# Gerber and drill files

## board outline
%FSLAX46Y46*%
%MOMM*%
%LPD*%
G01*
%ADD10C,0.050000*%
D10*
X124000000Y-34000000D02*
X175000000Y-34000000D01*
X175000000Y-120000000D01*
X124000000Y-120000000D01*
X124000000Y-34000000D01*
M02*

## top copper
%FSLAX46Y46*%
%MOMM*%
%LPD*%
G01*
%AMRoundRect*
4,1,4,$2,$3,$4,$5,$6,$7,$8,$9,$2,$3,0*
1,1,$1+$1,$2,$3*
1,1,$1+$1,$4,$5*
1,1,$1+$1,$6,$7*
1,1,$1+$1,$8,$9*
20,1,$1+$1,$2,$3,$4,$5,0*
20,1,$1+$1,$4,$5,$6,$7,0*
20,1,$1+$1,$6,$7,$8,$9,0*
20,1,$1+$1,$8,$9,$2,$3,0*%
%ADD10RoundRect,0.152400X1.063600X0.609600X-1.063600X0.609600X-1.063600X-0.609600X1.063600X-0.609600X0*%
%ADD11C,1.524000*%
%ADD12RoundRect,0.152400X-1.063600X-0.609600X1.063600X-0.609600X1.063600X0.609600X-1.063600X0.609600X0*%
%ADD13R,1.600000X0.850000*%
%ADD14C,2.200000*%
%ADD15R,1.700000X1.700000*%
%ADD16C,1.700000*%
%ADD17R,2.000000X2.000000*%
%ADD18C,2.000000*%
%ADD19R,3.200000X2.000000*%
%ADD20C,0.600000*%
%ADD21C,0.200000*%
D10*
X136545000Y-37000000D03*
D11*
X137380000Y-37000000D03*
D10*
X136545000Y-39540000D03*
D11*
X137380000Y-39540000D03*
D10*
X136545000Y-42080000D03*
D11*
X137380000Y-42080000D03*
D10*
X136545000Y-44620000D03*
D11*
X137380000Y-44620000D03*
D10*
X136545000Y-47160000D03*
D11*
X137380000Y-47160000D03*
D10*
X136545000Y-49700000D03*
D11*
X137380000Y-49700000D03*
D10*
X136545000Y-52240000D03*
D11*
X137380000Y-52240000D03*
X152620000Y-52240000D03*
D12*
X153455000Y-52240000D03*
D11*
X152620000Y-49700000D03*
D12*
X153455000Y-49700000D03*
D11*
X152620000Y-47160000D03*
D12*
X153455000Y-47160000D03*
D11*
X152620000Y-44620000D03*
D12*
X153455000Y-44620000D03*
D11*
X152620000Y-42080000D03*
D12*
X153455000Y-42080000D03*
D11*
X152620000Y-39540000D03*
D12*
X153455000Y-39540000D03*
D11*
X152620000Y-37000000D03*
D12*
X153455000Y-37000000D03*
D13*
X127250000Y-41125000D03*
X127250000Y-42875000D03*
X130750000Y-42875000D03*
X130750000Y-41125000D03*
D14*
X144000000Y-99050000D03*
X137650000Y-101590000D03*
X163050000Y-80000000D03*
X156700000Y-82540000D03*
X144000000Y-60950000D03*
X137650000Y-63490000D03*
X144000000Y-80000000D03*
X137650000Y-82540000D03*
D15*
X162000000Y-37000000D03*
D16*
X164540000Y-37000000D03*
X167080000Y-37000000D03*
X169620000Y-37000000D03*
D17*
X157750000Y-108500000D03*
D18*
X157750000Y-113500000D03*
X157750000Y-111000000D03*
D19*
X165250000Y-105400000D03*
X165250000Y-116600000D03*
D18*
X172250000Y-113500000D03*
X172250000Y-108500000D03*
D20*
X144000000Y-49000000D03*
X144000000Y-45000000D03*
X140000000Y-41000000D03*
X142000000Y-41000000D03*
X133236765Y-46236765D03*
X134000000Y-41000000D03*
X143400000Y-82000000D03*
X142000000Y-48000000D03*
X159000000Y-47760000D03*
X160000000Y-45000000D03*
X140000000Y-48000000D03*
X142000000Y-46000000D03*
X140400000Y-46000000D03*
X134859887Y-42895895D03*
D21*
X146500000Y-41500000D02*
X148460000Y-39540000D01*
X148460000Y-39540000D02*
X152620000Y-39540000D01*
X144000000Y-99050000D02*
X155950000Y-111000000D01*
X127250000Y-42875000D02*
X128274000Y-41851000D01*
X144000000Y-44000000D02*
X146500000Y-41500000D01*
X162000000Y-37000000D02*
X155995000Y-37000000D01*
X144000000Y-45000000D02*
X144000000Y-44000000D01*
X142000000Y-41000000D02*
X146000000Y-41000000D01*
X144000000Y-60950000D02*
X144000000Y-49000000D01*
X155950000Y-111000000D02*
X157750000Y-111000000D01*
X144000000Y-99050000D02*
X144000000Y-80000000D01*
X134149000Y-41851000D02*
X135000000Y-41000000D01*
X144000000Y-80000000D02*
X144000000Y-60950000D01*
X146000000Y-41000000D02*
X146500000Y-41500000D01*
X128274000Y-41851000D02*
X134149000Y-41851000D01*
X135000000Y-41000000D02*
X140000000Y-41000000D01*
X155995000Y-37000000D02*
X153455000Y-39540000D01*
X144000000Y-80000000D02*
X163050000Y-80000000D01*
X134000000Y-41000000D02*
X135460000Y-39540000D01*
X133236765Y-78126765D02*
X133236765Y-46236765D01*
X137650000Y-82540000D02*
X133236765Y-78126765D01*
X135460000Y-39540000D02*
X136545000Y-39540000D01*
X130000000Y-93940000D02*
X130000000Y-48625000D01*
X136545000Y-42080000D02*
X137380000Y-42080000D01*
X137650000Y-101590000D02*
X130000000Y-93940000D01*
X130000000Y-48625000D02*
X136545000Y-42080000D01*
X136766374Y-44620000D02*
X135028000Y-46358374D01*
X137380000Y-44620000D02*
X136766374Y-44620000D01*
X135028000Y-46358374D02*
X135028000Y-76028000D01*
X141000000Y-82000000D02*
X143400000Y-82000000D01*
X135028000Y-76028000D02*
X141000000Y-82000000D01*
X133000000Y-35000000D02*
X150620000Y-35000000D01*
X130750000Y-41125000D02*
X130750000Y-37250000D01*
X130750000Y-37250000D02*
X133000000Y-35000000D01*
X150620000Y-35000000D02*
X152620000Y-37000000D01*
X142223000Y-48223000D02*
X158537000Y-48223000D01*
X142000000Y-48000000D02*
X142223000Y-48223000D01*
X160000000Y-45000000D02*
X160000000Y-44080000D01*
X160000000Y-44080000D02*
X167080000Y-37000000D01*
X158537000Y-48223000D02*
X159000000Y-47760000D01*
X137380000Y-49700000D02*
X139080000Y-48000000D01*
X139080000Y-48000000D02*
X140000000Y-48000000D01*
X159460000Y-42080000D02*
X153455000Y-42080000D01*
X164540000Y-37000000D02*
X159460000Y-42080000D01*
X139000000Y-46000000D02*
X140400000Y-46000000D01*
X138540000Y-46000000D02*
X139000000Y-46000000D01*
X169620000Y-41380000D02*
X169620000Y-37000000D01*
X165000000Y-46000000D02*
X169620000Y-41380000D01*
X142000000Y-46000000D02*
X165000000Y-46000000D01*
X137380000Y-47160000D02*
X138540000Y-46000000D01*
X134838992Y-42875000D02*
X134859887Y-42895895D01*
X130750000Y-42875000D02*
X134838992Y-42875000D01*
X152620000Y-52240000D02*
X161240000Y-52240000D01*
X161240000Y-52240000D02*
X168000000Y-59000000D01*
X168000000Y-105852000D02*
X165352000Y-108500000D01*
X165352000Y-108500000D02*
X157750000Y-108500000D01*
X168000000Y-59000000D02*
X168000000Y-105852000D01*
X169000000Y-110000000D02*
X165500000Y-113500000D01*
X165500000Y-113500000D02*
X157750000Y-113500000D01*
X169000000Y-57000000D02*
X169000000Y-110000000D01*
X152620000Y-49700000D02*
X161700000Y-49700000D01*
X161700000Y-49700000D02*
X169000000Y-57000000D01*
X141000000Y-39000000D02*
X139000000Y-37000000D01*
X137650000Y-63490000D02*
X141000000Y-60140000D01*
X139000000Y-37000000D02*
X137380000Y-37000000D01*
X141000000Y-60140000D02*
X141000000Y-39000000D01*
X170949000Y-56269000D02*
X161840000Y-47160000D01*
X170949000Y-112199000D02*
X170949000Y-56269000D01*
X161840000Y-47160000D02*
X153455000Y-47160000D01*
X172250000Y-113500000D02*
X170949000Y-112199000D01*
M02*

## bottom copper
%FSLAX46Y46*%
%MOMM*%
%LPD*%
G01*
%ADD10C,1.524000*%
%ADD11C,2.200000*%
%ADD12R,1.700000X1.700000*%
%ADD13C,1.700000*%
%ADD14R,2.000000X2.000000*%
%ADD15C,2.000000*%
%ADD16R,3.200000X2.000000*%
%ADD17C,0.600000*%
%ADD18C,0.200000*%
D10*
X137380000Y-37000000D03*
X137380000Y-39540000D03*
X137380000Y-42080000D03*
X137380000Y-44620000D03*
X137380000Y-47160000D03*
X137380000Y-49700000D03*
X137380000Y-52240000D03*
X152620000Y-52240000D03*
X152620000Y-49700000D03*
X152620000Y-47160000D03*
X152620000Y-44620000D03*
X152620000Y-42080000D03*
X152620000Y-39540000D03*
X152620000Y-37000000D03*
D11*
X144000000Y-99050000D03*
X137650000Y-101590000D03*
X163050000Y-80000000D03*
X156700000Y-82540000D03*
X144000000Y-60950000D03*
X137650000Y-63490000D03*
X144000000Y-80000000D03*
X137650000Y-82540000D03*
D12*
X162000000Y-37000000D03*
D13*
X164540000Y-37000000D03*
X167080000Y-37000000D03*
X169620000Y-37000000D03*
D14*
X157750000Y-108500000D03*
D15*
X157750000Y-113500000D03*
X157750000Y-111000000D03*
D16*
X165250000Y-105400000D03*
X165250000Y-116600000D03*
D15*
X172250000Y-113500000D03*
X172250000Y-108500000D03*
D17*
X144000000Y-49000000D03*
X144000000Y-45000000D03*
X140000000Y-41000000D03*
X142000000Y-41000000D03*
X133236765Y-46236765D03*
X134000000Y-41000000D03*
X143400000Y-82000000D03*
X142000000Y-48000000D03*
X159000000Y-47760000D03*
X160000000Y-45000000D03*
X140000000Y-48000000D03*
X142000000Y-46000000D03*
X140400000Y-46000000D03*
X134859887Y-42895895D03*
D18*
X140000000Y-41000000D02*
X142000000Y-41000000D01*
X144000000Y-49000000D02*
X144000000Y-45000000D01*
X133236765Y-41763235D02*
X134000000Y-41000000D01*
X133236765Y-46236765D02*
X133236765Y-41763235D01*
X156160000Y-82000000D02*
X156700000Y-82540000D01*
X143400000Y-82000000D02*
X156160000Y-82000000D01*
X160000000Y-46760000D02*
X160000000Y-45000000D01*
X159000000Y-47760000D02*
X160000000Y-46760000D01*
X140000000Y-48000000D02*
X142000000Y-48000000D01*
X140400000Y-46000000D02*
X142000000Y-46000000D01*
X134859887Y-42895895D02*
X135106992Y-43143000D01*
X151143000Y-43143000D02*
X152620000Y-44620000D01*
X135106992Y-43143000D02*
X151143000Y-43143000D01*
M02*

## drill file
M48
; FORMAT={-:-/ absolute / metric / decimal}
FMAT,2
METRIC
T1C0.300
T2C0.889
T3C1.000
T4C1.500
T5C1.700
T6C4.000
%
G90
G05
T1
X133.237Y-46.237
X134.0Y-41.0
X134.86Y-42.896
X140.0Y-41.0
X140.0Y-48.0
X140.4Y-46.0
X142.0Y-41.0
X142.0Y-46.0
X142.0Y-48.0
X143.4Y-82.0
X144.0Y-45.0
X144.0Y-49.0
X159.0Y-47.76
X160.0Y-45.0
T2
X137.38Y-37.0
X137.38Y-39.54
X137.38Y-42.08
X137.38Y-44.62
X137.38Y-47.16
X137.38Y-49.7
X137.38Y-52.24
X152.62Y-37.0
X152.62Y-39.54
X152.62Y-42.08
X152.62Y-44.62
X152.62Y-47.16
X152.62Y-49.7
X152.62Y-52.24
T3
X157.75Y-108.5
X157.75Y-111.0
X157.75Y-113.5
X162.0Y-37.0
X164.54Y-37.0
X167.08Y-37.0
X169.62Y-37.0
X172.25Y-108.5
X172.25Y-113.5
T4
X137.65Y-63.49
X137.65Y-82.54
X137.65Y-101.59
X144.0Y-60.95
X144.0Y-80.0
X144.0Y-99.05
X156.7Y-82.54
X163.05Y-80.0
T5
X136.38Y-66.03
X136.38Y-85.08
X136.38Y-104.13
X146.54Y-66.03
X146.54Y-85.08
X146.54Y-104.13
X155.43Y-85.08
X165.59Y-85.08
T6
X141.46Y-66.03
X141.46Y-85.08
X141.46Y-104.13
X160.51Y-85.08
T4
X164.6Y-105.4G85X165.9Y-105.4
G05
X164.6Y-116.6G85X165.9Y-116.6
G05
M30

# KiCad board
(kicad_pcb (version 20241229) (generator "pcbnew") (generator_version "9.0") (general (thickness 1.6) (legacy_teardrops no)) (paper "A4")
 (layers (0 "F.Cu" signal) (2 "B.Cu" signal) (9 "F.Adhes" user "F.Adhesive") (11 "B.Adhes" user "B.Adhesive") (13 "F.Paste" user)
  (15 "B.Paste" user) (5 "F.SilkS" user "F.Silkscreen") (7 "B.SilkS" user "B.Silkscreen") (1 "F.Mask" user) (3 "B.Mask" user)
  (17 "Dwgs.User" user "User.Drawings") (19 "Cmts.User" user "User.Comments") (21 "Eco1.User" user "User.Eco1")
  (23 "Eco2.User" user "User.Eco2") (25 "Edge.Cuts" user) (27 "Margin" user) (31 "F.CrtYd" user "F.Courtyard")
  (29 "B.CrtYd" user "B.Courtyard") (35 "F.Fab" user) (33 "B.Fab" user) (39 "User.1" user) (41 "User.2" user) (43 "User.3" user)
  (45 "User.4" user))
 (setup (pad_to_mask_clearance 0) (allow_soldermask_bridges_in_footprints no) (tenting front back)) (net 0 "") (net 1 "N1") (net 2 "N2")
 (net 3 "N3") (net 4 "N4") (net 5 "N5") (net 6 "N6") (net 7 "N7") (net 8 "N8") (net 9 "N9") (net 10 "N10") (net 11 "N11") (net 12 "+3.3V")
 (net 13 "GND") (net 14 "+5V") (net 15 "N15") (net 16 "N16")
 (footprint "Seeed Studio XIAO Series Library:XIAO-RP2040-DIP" (layer "F.Cu") (at 145 44.62)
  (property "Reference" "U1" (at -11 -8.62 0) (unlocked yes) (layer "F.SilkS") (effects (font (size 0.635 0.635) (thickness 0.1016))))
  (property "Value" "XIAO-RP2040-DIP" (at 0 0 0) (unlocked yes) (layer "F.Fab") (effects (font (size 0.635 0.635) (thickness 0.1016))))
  (pad "1" smd roundrect (at -8.455 -7.62 180) (size 2.432 1.524) (layers "F.Cu" "F.Mask") (roundrect_rratio 0.1) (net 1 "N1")
   (thermal_bridge_angle 45))
  (pad "1" thru_hole circle (at -7.62 -7.62 180) (size 1.524 1.524) (drill 0.889) (layers "*.Cu" "*.Mask") (remove_unused_layers no)
   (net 1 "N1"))
  (pad "2" smd roundrect (at -8.455 -5.08 180) (size 2.432 1.524) (layers "F.Cu" "F.Mask") (roundrect_rratio 0.1) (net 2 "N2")
   (thermal_bridge_angle 45))
  (pad "2" thru_hole circle (at -7.62 -5.08 180) (size 1.524 1.524) (drill 0.889) (layers "*.Cu" "*.Mask") (remove_unused_layers no)
   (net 2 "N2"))
  (pad "3" smd roundrect (at -8.455 -2.54 180) (size 2.432 1.524) (layers "F.Cu" "F.Mask") (roundrect_rratio 0.1) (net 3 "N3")
   (thermal_bridge_angle 45))
  (pad "3" thru_hole circle (at -7.62 -2.54 180) (size 1.524 1.524) (drill 0.889) (layers "*.Cu" "*.Mask") (remove_unused_layers no)
   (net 3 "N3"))
  (pad "4" smd roundrect (at -8.455 0 180) (size 2.432 1.524) (layers "F.Cu" "F.Mask") (roundrect_rratio 0.1) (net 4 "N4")
   (thermal_bridge_angle 45))
  (pad "4" thru_hole circle (at -7.62 0 180) (size 1.524 1.524) (drill 0.889) (layers "*.Cu" "*.Mask") (remove_unused_layers no)
   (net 4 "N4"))
  (pad "5" smd roundrect (at -8.455 2.54 180) (size 2.432 1.524) (layers "F.Cu" "F.Mask") (roundrect_rratio 0.1) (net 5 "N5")
   (thermal_bridge_angle 45))
  (pad "5" thru_hole circle (at -7.62 2.54 180) (size 1.524 1.524) (drill 0.889) (layers "*.Cu" "*.Mask") (remove_unused_layers no)
   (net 5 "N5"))
  (pad "6" smd roundrect (at -8.455 5.08 180) (size 2.432 1.524) (layers "F.Cu" "F.Mask") (roundrect_rratio 0.1) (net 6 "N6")
   (thermal_bridge_angle 45))
  (pad "6" thru_hole circle (at -7.62 5.08 180) (size 1.524 1.524) (drill 0.889) (layers "*.Cu" "*.Mask") (remove_unused_layers no)
   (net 6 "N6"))
  (pad "7" smd roundrect (at -8.455 7.62 180) (size 2.432 1.524) (layers "F.Cu" "F.Mask") (roundrect_rratio 0.1) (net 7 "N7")
   (thermal_bridge_angle 45))
  (pad "7" thru_hole circle (at -7.62 7.62 180) (size 1.524 1.524) (drill 0.889) (layers "*.Cu" "*.Mask") (remove_unused_layers no)
   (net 7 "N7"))
  (pad "8" thru_hole circle (at 7.62 7.62) (size 1.524 1.524) (drill 0.889) (layers "*.Cu" "*.Mask") (remove_unused_layers no) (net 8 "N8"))
  (pad "8" smd roundrect (at 8.455 7.62) (size 2.432 1.524) (layers "F.Cu" "F.Mask") (roundrect_rratio 0.1) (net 8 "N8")
   (thermal_bridge_angle 45))
  (pad "9" thru_hole circle (at 7.62 5.08) (size 1.524 1.524) (drill 0.889) (layers "*.Cu" "*.Mask") (remove_unused_layers no) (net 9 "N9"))
  (pad "9" smd roundrect (at 8.455 5.08) (size 2.432 1.524) (layers "F.Cu" "F.Mask") (roundrect_rratio 0.1) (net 9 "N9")
   (thermal_bridge_angle 45))
  (pad "10" thru_hole circle (at 7.62 2.54) (size 1.524 1.524) (drill 0.889) (layers "*.Cu" "*.Mask") (remove_unused_layers no)
   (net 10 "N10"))
  (pad "10" smd roundrect (at 8.455 2.54) (size 2.432 1.524) (layers "F.Cu" "F.Mask") (roundrect_rratio 0.1) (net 10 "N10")
   (thermal_bridge_angle 45))
  (pad "11" thru_hole circle (at 7.62 0) (size 1.524 1.524) (drill 0.889) (layers "*.Cu" "*.Mask") (remove_unused_layers no) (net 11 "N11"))
  (pad "11" smd roundrect (at 8.455 0) (size 2.432 1.524) (layers "F.Cu" "F.Mask") (roundrect_rratio 0.1) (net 11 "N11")
   (thermal_bridge_angle 45))
  (pad "12" thru_hole circle (at 7.62 -2.54) (size 1.524 1.524) (drill 0.889) (layers "*.Cu" "*.Mask") (remove_unused_layers no)
   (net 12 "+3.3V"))
  (pad "12" smd roundrect (at 8.455 -2.54) (size 2.432 1.524) (layers "F.Cu" "F.Mask") (roundrect_rratio 0.1) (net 12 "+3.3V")
   (thermal_bridge_angle 45))
  (pad "13" thru_hole circle (at 7.62 -5.08) (size 1.524 1.524) (drill 0.889) (layers "*.Cu" "*.Mask") (remove_unused_layers no)
   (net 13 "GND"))
  (pad "13" smd roundrect (at 8.455 -5.08) (size 2.432 1.524) (layers "F.Cu" "F.Mask") (roundrect_rratio 0.1) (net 13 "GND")
   (thermal_bridge_angle 45))
  (pad "14" thru_hole circle (at 7.62 -7.62) (size 1.524 1.524) (drill 0.889) (layers "*.Cu" "*.Mask") (remove_unused_layers no)
   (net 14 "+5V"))
  (pad "14" smd roundrect (at 8.455 -7.62) (size 2.432 1.524) (layers "F.Cu" "F.Mask") (roundrect_rratio 0.1) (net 14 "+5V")
   (thermal_bridge_angle 45)))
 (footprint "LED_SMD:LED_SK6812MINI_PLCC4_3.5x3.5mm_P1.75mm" (layer "F.Cu") (at 129 42)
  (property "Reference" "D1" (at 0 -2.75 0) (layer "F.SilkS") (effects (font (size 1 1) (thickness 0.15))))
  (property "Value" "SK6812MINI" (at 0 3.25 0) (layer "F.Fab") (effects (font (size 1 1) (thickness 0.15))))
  (pad "1" smd rect (at -1.75 -0.875) (size 1.6 0.85) (layers "F.Cu" "F.Mask" "F.Paste") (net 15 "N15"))
  (pad "2" smd rect (at -1.75 0.875) (size 1.6 0.85) (layers "F.Cu" "F.Mask" "F.Paste") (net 13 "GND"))
  (pad "3" smd rect (at 1.75 0.875) (size 1.6 0.85) (layers "F.Cu" "F.Mask" "F.Paste") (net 11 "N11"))
  (pad "4" smd rect (at 1.75 -0.875) (size 1.6 0.85) (layers "F.Cu" "F.Mask" "F.Paste") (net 14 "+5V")))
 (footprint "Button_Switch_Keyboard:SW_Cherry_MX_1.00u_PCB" (layer "F.Cu") (at 144 99.05)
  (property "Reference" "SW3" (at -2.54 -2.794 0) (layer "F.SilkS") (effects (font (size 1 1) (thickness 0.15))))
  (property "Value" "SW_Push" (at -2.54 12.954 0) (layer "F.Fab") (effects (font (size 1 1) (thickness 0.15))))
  (pad "" np_thru_hole circle (at -7.62 5.08) (size 1.7 1.7) (drill 1.7) (layers "*.Cu" "*.Mask"))
  (pad "" np_thru_hole circle (at -2.54 5.08) (size 4 4) (drill 4) (layers "*.Cu" "*.Mask"))
  (pad "" np_thru_hole circle (at 2.54 5.08) (size 1.7 1.7) (drill 1.7) (layers "*.Cu" "*.Mask"))
  (pad "1" thru_hole circle (at 0 0) (size 2.2 2.2) (drill 1.5) (layers "*.Cu" "*.Mask") (remove_unused_layers no) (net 13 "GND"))
  (pad "2" thru_hole circle (at -6.35 2.54) (size 2.2 2.2) (drill 1.5) (layers "*.Cu" "*.Mask") (remove_unused_layers no) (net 3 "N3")))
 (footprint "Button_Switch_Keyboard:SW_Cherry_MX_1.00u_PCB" (layer "F.Cu") (at 163.05 80)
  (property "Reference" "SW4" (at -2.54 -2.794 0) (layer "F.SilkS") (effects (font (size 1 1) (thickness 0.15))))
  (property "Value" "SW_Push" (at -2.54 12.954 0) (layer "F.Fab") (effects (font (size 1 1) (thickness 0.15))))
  (pad "" np_thru_hole circle (at -7.62 5.08) (size 1.7 1.7) (drill 1.7) (layers "*.Cu" "*.Mask"))
  (pad "" np_thru_hole circle (at -2.54 5.08) (size 4 4) (drill 4) (layers "*.Cu" "*.Mask"))
  (pad "" np_thru_hole circle (at 2.54 5.08) (size 1.7 1.7) (drill 1.7) (layers "*.Cu" "*.Mask"))
  (pad "1" thru_hole circle (at 0 0) (size 2.2 2.2) (drill 1.5) (layers "*.Cu" "*.Mask") (remove_unused_layers no) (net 13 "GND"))
  (pad "2" thru_hole circle (at -6.35 2.54) (size 2.2 2.2) (drill 1.5) (layers "*.Cu" "*.Mask") (remove_unused_layers no) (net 4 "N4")))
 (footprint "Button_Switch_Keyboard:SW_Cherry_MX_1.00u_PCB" (layer "F.Cu") (at 144 60.95)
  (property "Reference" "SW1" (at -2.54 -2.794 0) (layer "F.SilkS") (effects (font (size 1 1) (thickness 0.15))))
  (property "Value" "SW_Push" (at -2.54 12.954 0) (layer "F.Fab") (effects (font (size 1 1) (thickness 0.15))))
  (pad "" np_thru_hole circle (at -7.62 5.08) (size 1.7 1.7) (drill 1.7) (layers "*.Cu" "*.Mask"))
  (pad "" np_thru_hole circle (at -2.54 5.08) (size 4 4) (drill 4) (layers "*.Cu" "*.Mask"))
  (pad "" np_thru_hole circle (at 2.54 5.08) (size 1.7 1.7) (drill 1.7) (layers "*.Cu" "*.Mask"))
  (pad "1" thru_hole circle (at 0 0) (size 2.2 2.2) (drill 1.5) (layers "*.Cu" "*.Mask") (remove_unused_layers no) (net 13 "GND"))
  (pad "2" thru_hole circle (at -6.35 2.54) (size 2.2 2.2) (drill 1.5) (layers "*.Cu" "*.Mask") (remove_unused_layers no) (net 1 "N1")))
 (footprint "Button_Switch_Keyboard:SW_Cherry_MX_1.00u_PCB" (layer "F.Cu") (at 144 80)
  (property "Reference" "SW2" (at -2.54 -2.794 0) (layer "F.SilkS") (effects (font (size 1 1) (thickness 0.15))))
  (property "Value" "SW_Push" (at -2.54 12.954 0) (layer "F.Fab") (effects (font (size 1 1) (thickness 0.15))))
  (pad "" np_thru_hole circle (at -7.62 5.08) (size 1.7 1.7) (drill 1.7) (layers "*.Cu" "*.Mask"))
  (pad "" np_thru_hole circle (at -2.54 5.08) (size 4 4) (drill 4) (layers "*.Cu" "*.Mask"))
  (pad "" np_thru_hole circle (at 2.54 5.08) (size 1.7 1.7) (drill 1.7) (layers "*.Cu" "*.Mask"))
  (pad "1" thru_hole circle (at 0 0) (size 2.2 2.2) (drill 1.5) (layers "*.Cu" "*.Mask") (remove_unused_layers no) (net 13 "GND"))
  (pad "2" thru_hole circle (at -6.35 2.54) (size 2.2 2.2) (drill 1.5) (layers "*.Cu" "*.Mask") (remove_unused_layers no) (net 2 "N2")))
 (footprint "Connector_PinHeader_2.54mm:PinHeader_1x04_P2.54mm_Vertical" (layer "F.Cu") (at 162 37 90)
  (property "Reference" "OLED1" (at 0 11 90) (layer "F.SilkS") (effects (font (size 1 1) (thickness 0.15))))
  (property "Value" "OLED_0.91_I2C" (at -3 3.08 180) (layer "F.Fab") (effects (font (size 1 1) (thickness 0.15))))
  (pad "1" thru_hole rect (at 0 0 90) (size 1.7 1.7) (drill 1) (layers "*.Cu" "*.Mask") (remove_unused_layers no) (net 13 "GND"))
  (pad "2" thru_hole circle (at 0 2.54 90) (size 1.7 1.7) (drill 1) (layers "*.Cu" "*.Mask") (remove_unused_layers no) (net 12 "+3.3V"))
  (pad "3" thru_hole circle (at 0 5.08 90) (size 1.7 1.7) (drill 1) (layers "*.Cu" "*.Mask") (remove_unused_layers no) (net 6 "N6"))
  (pad "4" thru_hole circle (at 0 7.62 90) (size 1.7 1.7) (drill 1) (layers "*.Cu" "*.Mask") (remove_unused_layers no) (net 5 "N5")))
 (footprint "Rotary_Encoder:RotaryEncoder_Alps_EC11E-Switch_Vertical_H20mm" (layer "F.Cu") (at 157.75 108.5)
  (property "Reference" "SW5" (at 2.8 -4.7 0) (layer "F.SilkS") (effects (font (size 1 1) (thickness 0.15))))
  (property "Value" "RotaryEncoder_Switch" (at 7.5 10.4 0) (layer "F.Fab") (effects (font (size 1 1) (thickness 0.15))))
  (pad "A" thru_hole rect (at 0 0) (size 2 2) (drill 1) (layers "*.Cu" "*.Mask") (remove_unused_layers no) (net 8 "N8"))
  (pad "B" thru_hole circle (at 0 5) (size 2 2) (drill 1) (layers "*.Cu" "*.Mask") (remove_unused_layers no) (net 9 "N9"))
  (pad "C" thru_hole circle (at 0 2.5) (size 2 2) (drill 1) (layers "*.Cu" "*.Mask") (remove_unused_layers no) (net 13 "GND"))
  (pad "MP" thru_hole rect (at 7.5 -3.1) (size 3.2 2) (drill oval 2.8 1.5) (layers "*.Cu" "*.Mask") (remove_unused_layers no))
  (pad "MP" thru_hole rect (at 7.5 8.1) (size 3.2 2) (drill oval 2.8 1.5) (layers "*.Cu" "*.Mask") (remove_unused_layers no))
  (pad "S1" thru_hole circle (at 14.5 5) (size 2 2) (drill 1) (layers "*.Cu" "*.Mask") (remove_unused_layers no) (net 10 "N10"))
  (pad "S2" thru_hole circle (at 14.5 0) (size 2 2) (drill 1) (layers "*.Cu" "*.Mask") (remove_unused_layers no) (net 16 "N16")))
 (gr_rect (start 124 34) (end 175 120) (stroke (width 0.05) (type default)) (fill no) (layer "Edge.Cuts"))
 (segment (start 146.5 41.5) (end 148.46 39.54) (width 0.2) (layer "F.Cu") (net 13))
 (segment (start 148.46 39.54) (end 152.62 39.54) (width 0.2) (layer "F.Cu") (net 13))
 (segment (start 144 99.05) (end 155.95 111) (width 0.2) (layer "F.Cu") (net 13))
 (segment (start 127.25 42.875) (end 128.274 41.851) (width 0.2) (layer "F.Cu") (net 13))
 (segment (start 144 44) (end 146.5 41.5) (width 0.2) (layer "F.Cu") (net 13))
 (segment (start 162 37) (end 155.995 37) (width 0.2) (layer "F.Cu") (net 13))
 (segment (start 144 45) (end 144 44) (width 0.2) (layer "F.Cu") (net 13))
 (segment (start 142 41) (end 146 41) (width 0.2) (layer "F.Cu") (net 13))
 (segment (start 144 60.95) (end 144 49) (width 0.2) (layer "F.Cu") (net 13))
 (segment (start 155.95 111) (end 157.75 111) (width 0.2) (layer "F.Cu") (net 13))
 (segment (start 144 99.05) (end 144 80) (width 0.2) (layer "F.Cu") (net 13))
 (segment (start 134.149 41.851) (end 135 41) (width 0.2) (layer "F.Cu") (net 13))
 (segment (start 144 80) (end 144 60.95) (width 0.2) (layer "F.Cu") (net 13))
 (segment (start 146 41) (end 146.5 41.5) (width 0.2) (layer "F.Cu") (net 13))
 (segment (start 128.274 41.851) (end 134.149 41.851) (width 0.2) (layer "F.Cu") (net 13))
 (segment (start 135 41) (end 140 41) (width 0.2) (layer "F.Cu") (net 13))
 (segment (start 155.995 37) (end 153.455 39.54) (width 0.2) (layer "F.Cu") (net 13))
 (segment (start 144 80) (end 163.05 80) (width 0.2) (layer "F.Cu") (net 13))
 (via (at 144 49) (size 0.6) (drill 0.3) (layers "F.Cu" "B.Cu") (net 13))
 (via (at 144 45) (size 0.6) (drill 0.3) (layers "F.Cu" "B.Cu") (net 13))
 (via (at 140 41) (size 0.6) (drill 0.3) (layers "F.Cu" "B.Cu") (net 13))
 (via (at 142 41) (size 0.6) (drill 0.3) (layers "F.Cu" "B.Cu") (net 13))
 (segment (start 140 41) (end 142 41) (width 0.2) (layer "B.Cu") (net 13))
 (segment (start 144 49) (end 144 45) (width 0.2) (layer "B.Cu") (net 13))
 (segment (start 134 41) (end 135.46 39.54) (width 0.2) (layer "F.Cu") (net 2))
 (segment (start 133.236765 78.126765) (end 133.236765 46.236765) (width 0.2) (layer "F.Cu") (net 2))
 (segment (start 137.65 82.54) (end 133.236765 78.126765) (width 0.2) (layer "F.Cu") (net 2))
 (segment (start 135.46 39.54) (end 136.545 39.54) (width 0.2) (layer "F.Cu") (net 2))
 (via (at 133.236765 46.236765) (size 0.6) (drill 0.3) (layers "F.Cu" "B.Cu") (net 2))
 (via (at 134 41) (size 0.6) (drill 0.3) (layers "F.Cu" "B.Cu") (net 2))
 (segment (start 133.236765 41.763235) (end 134 41) (width 0.2) (layer "B.Cu") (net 2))
 (segment (start 133.236765 46.236765) (end 133.236765 41.763235) (width 0.2) (layer "B.Cu") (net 2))
 (segment (start 130 93.94) (end 130 48.625) (width 0.2) (layer "F.Cu") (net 3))
 (segment (start 136.545 42.08) (end 137.38 42.08) (width 0.2) (layer "F.Cu") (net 3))
 (segment (start 137.65 101.59) (end 130 93.94) (width 0.2) (layer "F.Cu") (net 3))
 (segment (start 130 48.625) (end 136.545 42.08) (width 0.2) (layer "F.Cu") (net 3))
 (segment (start 136.766374 44.62) (end 135.028 46.358374) (width 0.2) (layer "F.Cu") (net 4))
 (segment (start 137.38 44.62) (end 136.766374 44.62) (width 0.2) (layer "F.Cu") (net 4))
 (segment (start 135.028 46.358374) (end 135.028 76.028) (width 0.2) (layer "F.Cu") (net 4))
 (segment (start 141 82) (end 143.4 82) (width 0.2) (layer "F.Cu") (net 4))
 (segment (start 135.028 76.028) (end 141 82) (width 0.2) (layer "F.Cu") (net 4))
 (via (at 143.4 82) (size 0.6) (drill 0.3) (layers "F.Cu" "B.Cu") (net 4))
 (segment (start 156.16 82) (end 156.7 82.54) (width 0.2) (layer "B.Cu") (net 4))
 (segment (start 143.4 82) (end 156.16 82) (width 0.2) (layer "B.Cu") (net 4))
 (segment (start 133 35) (end 150.62 35) (width 0.2) (layer "F.Cu") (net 14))
 (segment (start 130.75 41.125) (end 130.75 37.25) (width 0.2) (layer "F.Cu") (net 14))
 (segment (start 130.75 37.25) (end 133 35) (width 0.2) (layer "F.Cu") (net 14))
 (segment (start 150.62 35) (end 152.62 37) (width 0.2) (layer "F.Cu") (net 14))
 (segment (start 142.223 48.223) (end 158.537 48.223) (width 0.2) (layer "F.Cu") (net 6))
 (segment (start 142 48) (end 142.223 48.223) (width 0.2) (layer "F.Cu") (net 6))
 (segment (start 160 45) (end 160 44.08) (width 0.2) (layer "F.Cu") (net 6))
 (segment (start 160 44.08) (end 167.08 37) (width 0.2) (layer "F.Cu") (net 6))
 (segment (start 158.537 48.223) (end 159 47.76) (width 0.2) (layer "F.Cu") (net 6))
 (segment (start 137.38 49.7) (end 139.08 48) (width 0.2) (layer "F.Cu") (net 6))
 (segment (start 139.08 48) (end 140 48) (width 0.2) (layer "F.Cu") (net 6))
 (via (at 142 48) (size 0.6) (drill 0.3) (layers "F.Cu" "B.Cu") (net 6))
 (via (at 159 47.76) (size 0.6) (drill 0.3) (layers "F.Cu" "B.Cu") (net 6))
 (via (at 160 45) (size 0.6) (drill 0.3) (layers "F.Cu" "B.Cu") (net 6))
 (via (at 140 48) (size 0.6) (drill 0.3) (layers "F.Cu" "B.Cu") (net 6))
 (segment (start 160 46.76) (end 160 45) (width 0.2) (layer "B.Cu") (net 6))
 (segment (start 159 47.76) (end 160 46.76) (width 0.2) (layer "B.Cu") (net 6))
 (segment (start 140 48) (end 142 48) (width 0.2) (layer "B.Cu") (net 6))
 (segment (start 159.46 42.08) (end 153.455 42.08) (width 0.2) (layer "F.Cu") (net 12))
 (segment (start 164.54 37) (end 159.46 42.08) (width 0.2) (layer "F.Cu") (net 12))
 (segment (start 139 46) (end 140.4 46) (width 0.2) (layer "F.Cu") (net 5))
 (segment (start 138.54 46) (end 139 46) (width 0.2) (layer "F.Cu") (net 5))
 (segment (start 169.62 41.38) (end 169.62 37) (width 0.2) (layer "F.Cu") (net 5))
 (segment (start 165 46) (end 169.62 41.38) (width 0.2) (layer "F.Cu") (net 5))
 (segment (start 142 46) (end 165 46) (width 0.2) (layer "F.Cu") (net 5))
 (segment (start 137.38 47.16) (end 138.54 46) (width 0.2) (layer "F.Cu") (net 5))
 (via (at 142 46) (size 0.6) (drill 0.3) (layers "F.Cu" "B.Cu") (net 5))
 (via (at 140.4 46) (size 0.6) (drill 0.3) (layers "F.Cu" "B.Cu") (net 5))
 (segment (start 140.4 46) (end 142 46) (width 0.2) (layer "B.Cu") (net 5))
 (segment (start 134.838992 42.875) (end 134.859887 42.895895) (width 0.2) (layer "F.Cu") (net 11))
 (segment (start 130.75 42.875) (end 134.838992 42.875) (width 0.2) (layer "F.Cu") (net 11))
 (via (at 134.859887 42.895895) (size 0.6) (drill 0.3) (layers "F.Cu" "B.Cu") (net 11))
 (segment (start 134.859887 42.895895) (end 135.106992 43.143) (width 0.2) (layer "B.Cu") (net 11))
 (segment (start 151.143 43.143) (end 152.62 44.62) (width 0.2) (layer "B.Cu") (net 11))
 (segment (start 135.106992 43.143) (end 151.143 43.143) (width 0.2) (layer "B.Cu") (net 11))
 (segment (start 152.62 52.24) (end 161.24 52.24) (width 0.2) (layer "F.Cu") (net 8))
 (segment (start 161.24 52.24) (end 168 59) (width 0.2) (layer "F.Cu") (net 8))
 (segment (start 168 105.852) (end 165.352 108.5) (width 0.2) (layer "F.Cu") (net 8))
 (segment (start 165.352 108.5) (end 157.75 108.5) (width 0.2) (layer "F.Cu") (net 8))
 (segment (start 168 59) (end 168 105.852) (width 0.2) (layer "F.Cu") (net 8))
 (segment (start 169 110) (end 165.5 113.5) (width 0.2) (layer "F.Cu") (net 9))
 (segment (start 165.5 113.5) (end 157.75 113.5) (width 0.2) (layer "F.Cu") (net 9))
 (segment (start 169 57) (end 169 110) (width 0.2) (layer "F.Cu") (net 9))
 (segment (start 152.62 49.7) (end 161.7 49.7) (width 0.2) (layer "F.Cu") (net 9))
 (segment (start 161.7 49.7) (end 169 57) (width 0.2) (layer "F.Cu") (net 9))
 (segment (start 141 39) (end 139 37) (width 0.2) (layer "F.Cu") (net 1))
 (segment (start 137.65 63.49) (end 141 60.14) (width 0.2) (layer "F.Cu") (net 1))
 (segment (start 139 37) (end 137.38 37) (width 0.2) (layer "F.Cu") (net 1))
 (segment (start 141 60.14) (end 141 39) (width 0.2) (layer "F.Cu") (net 1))
 (segment (start 170.949 56.269) (end 161.84 47.16) (width 0.2) (layer "F.Cu") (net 10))
 (segment (start 170.949 112.199) (end 170.949 56.269) (width 0.2) (layer "F.Cu") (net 10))
 (segment (start 161.84 47.16) (end 153.455 47.16) (width 0.2) (layer "F.Cu") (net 10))
 (segment (start 172.25 113.5) (end 170.949 112.199) (width 0.2) (layer "F.Cu") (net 10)))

